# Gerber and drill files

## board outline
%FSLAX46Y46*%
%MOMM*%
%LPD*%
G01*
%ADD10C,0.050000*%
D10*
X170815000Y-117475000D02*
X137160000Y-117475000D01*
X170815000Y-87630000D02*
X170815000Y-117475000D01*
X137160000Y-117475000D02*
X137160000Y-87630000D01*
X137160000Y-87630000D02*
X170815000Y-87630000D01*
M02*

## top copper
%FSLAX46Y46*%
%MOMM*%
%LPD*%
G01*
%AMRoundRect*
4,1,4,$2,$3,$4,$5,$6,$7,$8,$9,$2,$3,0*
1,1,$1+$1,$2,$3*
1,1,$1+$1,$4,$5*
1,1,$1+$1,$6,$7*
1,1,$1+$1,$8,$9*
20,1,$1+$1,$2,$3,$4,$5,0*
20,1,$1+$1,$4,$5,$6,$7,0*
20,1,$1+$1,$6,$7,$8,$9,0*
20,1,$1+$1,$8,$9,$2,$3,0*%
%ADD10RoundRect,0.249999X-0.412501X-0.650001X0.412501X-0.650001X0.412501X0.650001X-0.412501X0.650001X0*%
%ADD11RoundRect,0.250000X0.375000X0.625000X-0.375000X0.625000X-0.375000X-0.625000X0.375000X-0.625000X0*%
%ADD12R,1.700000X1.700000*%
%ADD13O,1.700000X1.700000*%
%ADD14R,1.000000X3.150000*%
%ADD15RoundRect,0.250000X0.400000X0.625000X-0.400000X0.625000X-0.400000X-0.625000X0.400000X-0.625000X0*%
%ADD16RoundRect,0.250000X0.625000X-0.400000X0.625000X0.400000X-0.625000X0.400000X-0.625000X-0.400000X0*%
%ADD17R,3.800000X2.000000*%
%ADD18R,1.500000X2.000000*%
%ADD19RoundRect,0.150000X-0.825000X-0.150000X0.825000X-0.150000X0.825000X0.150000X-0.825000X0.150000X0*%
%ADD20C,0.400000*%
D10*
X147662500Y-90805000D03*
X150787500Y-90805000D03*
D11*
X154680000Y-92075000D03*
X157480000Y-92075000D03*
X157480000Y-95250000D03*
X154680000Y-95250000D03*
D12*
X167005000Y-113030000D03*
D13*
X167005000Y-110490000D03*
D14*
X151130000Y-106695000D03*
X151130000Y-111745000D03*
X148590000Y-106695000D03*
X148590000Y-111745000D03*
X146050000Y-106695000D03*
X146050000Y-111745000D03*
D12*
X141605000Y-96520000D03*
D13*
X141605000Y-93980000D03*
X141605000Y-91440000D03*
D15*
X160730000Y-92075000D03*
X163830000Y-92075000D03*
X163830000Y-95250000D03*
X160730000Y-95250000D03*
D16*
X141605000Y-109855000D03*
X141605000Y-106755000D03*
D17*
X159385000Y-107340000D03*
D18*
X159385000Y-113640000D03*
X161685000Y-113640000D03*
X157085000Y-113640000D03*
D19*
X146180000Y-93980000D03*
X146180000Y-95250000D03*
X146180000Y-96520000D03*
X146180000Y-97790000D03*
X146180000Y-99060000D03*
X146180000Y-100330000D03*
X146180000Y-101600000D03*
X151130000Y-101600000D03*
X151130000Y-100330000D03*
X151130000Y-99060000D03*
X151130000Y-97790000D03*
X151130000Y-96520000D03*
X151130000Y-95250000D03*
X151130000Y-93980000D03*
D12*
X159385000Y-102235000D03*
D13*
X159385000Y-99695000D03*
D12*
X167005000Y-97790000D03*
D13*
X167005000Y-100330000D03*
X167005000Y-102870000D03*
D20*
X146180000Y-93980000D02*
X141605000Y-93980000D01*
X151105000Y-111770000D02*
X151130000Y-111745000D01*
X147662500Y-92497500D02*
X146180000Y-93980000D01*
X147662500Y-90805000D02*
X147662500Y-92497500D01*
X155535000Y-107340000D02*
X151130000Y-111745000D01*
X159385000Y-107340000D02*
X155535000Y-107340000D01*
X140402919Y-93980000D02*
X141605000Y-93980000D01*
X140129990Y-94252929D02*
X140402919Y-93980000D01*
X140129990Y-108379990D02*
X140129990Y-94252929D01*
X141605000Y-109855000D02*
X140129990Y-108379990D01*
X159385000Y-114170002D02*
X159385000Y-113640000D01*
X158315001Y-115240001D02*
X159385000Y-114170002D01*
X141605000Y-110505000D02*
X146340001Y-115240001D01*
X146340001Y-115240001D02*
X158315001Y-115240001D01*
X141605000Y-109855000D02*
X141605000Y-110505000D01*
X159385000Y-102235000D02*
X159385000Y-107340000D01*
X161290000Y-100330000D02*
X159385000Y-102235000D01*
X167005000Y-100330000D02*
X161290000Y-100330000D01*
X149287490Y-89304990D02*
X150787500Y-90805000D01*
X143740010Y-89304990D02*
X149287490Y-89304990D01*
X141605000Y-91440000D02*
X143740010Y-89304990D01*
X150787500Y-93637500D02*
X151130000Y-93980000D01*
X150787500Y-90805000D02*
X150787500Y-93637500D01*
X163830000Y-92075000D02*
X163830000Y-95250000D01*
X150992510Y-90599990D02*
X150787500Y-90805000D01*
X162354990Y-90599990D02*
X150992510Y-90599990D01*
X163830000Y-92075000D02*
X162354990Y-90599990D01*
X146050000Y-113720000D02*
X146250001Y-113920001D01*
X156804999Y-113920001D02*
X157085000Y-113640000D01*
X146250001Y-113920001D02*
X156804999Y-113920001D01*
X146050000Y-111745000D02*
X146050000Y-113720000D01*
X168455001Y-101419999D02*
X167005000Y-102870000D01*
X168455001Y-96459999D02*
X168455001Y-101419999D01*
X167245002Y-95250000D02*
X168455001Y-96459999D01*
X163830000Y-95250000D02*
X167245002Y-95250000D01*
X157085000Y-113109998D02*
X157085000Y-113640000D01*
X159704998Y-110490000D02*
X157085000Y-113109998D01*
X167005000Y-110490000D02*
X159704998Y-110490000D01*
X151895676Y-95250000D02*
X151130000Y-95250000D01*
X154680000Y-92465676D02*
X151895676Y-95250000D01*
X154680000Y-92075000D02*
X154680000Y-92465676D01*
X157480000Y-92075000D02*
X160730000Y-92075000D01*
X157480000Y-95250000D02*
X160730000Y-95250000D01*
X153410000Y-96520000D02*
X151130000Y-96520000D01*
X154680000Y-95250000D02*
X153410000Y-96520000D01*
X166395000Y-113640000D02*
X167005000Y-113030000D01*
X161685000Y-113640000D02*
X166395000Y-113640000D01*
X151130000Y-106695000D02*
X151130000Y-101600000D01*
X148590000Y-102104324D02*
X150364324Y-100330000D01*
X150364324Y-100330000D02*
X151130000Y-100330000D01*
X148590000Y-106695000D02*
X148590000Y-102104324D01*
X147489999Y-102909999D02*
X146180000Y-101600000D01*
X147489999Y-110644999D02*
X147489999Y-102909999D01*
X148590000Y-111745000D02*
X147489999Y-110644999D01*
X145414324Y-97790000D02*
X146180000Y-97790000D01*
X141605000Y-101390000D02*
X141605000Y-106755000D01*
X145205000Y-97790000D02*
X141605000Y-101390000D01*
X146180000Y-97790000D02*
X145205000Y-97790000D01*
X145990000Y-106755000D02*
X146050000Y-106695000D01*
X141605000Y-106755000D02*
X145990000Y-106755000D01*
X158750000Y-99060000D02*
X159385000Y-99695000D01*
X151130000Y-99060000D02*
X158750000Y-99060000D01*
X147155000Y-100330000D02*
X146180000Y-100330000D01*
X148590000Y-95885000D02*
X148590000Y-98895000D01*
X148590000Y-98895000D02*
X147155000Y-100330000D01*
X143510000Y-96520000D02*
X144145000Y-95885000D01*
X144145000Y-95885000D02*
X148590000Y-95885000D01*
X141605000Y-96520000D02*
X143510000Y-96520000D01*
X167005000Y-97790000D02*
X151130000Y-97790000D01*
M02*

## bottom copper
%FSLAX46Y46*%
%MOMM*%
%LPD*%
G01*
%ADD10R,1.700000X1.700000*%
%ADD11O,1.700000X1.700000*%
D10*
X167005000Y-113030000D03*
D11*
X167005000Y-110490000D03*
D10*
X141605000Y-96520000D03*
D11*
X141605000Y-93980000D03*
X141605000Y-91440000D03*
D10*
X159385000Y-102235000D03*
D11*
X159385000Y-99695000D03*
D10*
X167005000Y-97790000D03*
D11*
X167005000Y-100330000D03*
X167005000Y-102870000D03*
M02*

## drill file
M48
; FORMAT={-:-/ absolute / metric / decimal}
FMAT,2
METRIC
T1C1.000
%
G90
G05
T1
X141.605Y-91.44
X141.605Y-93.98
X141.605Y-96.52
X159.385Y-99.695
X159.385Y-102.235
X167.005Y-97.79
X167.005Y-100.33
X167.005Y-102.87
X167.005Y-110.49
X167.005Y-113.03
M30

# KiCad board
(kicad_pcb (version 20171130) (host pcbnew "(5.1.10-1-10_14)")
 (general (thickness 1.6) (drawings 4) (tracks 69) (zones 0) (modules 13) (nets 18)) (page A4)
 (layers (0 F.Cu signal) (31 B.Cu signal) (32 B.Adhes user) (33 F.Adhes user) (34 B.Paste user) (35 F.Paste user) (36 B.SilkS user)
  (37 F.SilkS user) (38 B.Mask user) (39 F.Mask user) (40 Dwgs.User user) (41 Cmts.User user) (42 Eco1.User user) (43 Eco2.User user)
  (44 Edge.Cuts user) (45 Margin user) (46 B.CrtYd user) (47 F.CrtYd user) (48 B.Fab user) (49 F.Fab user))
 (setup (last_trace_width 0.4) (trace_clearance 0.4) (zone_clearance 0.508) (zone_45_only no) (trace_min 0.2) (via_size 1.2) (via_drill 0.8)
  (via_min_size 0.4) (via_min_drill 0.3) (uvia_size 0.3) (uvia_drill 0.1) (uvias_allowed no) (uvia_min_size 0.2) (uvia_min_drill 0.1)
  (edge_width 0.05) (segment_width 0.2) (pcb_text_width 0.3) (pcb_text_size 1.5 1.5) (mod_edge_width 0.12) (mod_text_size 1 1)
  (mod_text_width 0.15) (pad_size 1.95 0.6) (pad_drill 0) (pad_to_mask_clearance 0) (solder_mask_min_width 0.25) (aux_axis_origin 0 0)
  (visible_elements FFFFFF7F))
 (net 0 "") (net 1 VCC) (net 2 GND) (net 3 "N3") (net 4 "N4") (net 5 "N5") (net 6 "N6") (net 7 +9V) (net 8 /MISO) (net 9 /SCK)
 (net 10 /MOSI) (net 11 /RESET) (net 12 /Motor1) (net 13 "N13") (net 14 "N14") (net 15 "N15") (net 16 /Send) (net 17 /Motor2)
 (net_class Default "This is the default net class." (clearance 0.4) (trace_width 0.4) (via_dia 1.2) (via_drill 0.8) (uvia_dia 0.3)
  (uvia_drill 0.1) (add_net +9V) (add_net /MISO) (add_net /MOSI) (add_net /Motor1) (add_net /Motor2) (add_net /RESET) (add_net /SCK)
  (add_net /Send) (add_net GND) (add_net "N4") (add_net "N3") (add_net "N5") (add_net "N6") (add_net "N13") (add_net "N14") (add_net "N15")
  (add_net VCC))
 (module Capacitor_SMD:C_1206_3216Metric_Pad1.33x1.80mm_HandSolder (layer F.Cu) (at 149.225 90.805)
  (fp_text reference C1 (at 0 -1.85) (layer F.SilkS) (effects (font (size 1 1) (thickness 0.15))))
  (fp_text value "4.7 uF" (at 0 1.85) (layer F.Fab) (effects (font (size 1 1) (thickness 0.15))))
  (pad 1 smd roundrect (at -1.5625 0) (size 1.325 1.8) (layers F.Cu F.Paste F.Mask) (roundrect_rratio 0.1886784905660377) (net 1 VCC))
  (pad 2 smd roundrect (at 1.5625 0) (size 1.325 1.8) (layers F.Cu F.Paste F.Mask) (roundrect_rratio 0.1886784905660377) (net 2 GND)))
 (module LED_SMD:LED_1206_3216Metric (layer F.Cu) (at 156.08 92.075 180)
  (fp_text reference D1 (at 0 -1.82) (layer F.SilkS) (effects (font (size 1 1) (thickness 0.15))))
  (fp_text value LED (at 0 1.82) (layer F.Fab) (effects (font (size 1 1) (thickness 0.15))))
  (pad 2 smd roundrect (at 1.4 0 180) (size 1.25 1.75) (layers F.Cu F.Paste F.Mask) (roundrect_rratio 0.2) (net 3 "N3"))
  (pad 1 smd roundrect (at -1.4 0 180) (size 1.25 1.75) (layers F.Cu F.Paste F.Mask) (roundrect_rratio 0.2) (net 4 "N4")))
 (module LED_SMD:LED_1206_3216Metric (layer F.Cu) (at 156.08 95.25 180)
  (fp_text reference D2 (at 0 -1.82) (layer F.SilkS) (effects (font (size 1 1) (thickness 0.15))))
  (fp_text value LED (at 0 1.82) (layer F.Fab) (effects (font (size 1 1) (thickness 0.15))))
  (pad 1 smd roundrect (at -1.4 0 180) (size 1.25 1.75) (layers F.Cu F.Paste F.Mask) (roundrect_rratio 0.2) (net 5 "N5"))
  (pad 2 smd roundrect (at 1.4 0 180) (size 1.25 1.75) (layers F.Cu F.Paste F.Mask) (roundrect_rratio 0.2) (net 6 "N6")))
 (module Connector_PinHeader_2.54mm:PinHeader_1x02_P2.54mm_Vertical (layer F.Cu) (at 167.005 113.03 180)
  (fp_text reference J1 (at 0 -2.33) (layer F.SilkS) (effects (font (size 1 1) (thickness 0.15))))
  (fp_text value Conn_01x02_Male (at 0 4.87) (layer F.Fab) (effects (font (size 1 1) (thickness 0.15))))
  (pad 1 thru_hole rect (at 0 0 180) (size 1.7 1.7) (drill 1) (layers *.Cu *.Mask) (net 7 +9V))
  (pad 2 thru_hole oval (at 0 2.54 180) (size 1.7 1.7) (drill 1) (layers *.Cu *.Mask) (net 2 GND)))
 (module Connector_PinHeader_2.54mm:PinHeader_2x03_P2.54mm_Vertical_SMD (layer F.Cu) (at 148.59 109.22 270)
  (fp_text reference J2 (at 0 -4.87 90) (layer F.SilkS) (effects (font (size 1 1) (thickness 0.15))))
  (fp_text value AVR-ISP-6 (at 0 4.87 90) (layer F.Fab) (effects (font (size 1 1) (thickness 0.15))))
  (pad 1 smd rect (at -2.525 -2.54 270) (size 3.15 1) (layers F.Cu F.Paste F.Mask) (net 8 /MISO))
  (pad 2 smd rect (at 2.525 -2.54 270) (size 3.15 1) (layers F.Cu F.Paste F.Mask) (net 1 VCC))
  (pad 3 smd rect (at -2.525 0 270) (size 3.15 1) (layers F.Cu F.Paste F.Mask) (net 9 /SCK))
  (pad 4 smd rect (at 2.525 0 270) (size 3.15 1) (layers F.Cu F.Paste F.Mask) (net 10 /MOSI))
  (pad 5 smd rect (at -2.525 2.54 270) (size 3.15 1) (layers F.Cu F.Paste F.Mask) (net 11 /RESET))
  (pad 6 smd rect (at 2.525 2.54 270) (size 3.15 1) (layers F.Cu F.Paste F.Mask) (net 2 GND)))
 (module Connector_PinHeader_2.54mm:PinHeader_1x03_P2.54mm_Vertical (layer F.Cu) (at 141.605 96.52 180)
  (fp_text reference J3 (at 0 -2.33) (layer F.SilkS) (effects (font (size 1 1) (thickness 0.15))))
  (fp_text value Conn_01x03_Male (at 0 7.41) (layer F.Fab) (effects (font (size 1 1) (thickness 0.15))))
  (pad 1 thru_hole rect (at 0 0 180) (size 1.7 1.7) (drill 1) (layers *.Cu *.Mask) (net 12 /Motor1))
  (pad 2 thru_hole oval (at 0 2.54 180) (size 1.7 1.7) (drill 1) (layers *.Cu *.Mask) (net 1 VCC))
  (pad 3 thru_hole oval (at 0 5.08 180) (size 1.7 1.7) (drill 1) (layers *.Cu *.Mask) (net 2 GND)))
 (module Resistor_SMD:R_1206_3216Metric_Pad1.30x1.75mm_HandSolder (layer F.Cu) (at 162.28 92.075 180)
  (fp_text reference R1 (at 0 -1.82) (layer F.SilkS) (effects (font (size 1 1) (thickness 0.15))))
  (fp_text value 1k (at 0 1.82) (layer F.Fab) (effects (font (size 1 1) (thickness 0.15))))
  (pad 2 smd roundrect (at 1.55 0 180) (size 1.3 1.75) (layers F.Cu F.Paste F.Mask) (roundrect_rratio 0.1923076923076923) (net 4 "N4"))
  (pad 1 smd roundrect (at -1.55 0 180) (size 1.3 1.75) (layers F.Cu F.Paste F.Mask) (roundrect_rratio 0.1923076923076923) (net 2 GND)))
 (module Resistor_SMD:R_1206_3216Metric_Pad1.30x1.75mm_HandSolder (layer F.Cu) (at 162.28 95.25 180)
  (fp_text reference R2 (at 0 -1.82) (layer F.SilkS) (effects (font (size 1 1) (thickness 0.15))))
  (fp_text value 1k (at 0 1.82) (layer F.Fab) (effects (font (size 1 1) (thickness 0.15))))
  (pad 1 smd roundrect (at -1.55 0 180) (size 1.3 1.75) (layers F.Cu F.Paste F.Mask) (roundrect_rratio 0.1923076923076923) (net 2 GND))
  (pad 2 smd roundrect (at 1.55 0 180) (size 1.3 1.75) (layers F.Cu F.Paste F.Mask) (roundrect_rratio 0.1923076923076923) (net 5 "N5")))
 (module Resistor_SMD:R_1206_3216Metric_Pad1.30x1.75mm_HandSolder (layer F.Cu) (at 141.605 108.305 90)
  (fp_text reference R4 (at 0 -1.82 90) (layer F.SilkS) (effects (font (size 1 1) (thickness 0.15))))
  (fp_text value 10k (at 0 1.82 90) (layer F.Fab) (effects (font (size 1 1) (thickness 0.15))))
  (pad 1 smd roundrect (at -1.55 0 90) (size 1.3 1.75) (layers F.Cu F.Paste F.Mask) (roundrect_rratio 0.1923076923076923) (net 1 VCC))
  (pad 2 smd roundrect (at 1.55 0 90) (size 1.3 1.75) (layers F.Cu F.Paste F.Mask) (roundrect_rratio 0.1923076923076923) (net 11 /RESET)))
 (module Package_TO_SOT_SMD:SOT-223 (layer F.Cu) (at 159.385 110.49 90)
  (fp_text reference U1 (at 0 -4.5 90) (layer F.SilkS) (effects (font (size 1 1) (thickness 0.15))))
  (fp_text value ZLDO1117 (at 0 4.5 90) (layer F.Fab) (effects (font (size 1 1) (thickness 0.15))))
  (pad 4 smd rect (at 3.15 0 90) (size 2 3.8) (layers F.Cu F.Paste F.Mask) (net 1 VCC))
  (pad 2 smd rect (at -3.15 0 90) (size 2 1.5) (layers F.Cu F.Paste F.Mask) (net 1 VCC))
  (pad 3 smd rect (at -3.15 2.3 90) (size 2 1.5) (layers F.Cu F.Paste F.Mask) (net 7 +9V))
  (pad 1 smd rect (at -3.15 -2.3 90) (size 2 1.5) (layers F.Cu F.Paste F.Mask) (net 2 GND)))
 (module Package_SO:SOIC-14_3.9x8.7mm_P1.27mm (layer F.Cu) (at 148.655 97.79)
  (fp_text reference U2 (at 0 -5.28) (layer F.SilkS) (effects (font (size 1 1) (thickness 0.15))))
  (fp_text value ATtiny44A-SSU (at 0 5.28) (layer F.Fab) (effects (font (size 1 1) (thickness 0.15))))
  (pad 1 smd roundrect (at -2.475 -3.81) (size 1.95 0.6) (layers F.Cu F.Paste F.Mask) (roundrect_rratio 0.25) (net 1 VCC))
  (pad 2 smd roundrect (at -2.475 -2.54) (size 1.95 0.6) (layers F.Cu F.Paste F.Mask) (roundrect_rratio 0.25) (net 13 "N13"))
  (pad 3 smd roundrect (at -2.475 -1.27) (size 1.95 0.6) (layers F.Cu F.Paste F.Mask) (roundrect_rratio 0.25) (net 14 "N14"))
  (pad 4 smd roundrect (at -2.475 0) (size 1.95 0.6) (layers F.Cu F.Paste F.Mask) (roundrect_rratio 0.25) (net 11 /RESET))
  (pad 5 smd roundrect (at -2.475 1.27) (size 1.95 0.6) (layers F.Cu F.Paste F.Mask) (roundrect_rratio 0.25) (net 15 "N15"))
  (pad 6 smd roundrect (at -2.475 2.54) (size 1.95 0.6) (layers F.Cu F.Paste F.Mask) (roundrect_rratio 0.25) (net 12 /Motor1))
  (pad 7 smd roundrect (at -2.475 3.81) (size 1.95 0.6) (layers F.Cu F.Paste F.Mask) (roundrect_rratio 0.25) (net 10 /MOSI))
  (pad 8 smd roundrect (at 2.475 3.81) (size 1.95 0.6) (layers F.Cu F.Paste F.Mask) (roundrect_rratio 0.25) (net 8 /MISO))
  (pad 9 smd roundrect (at 2.475 2.54) (size 1.95 0.6) (layers F.Cu F.Paste F.Mask) (roundrect_rratio 0.25) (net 9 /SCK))
  (pad 10 smd roundrect (at 2.475 1.27) (size 1.95 0.6) (layers F.Cu F.Paste F.Mask) (roundrect_rratio 0.25) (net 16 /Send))
  (pad 11 smd roundrect (at 2.475 0) (size 1.95 0.6) (layers F.Cu F.Paste F.Mask) (roundrect_rratio 0.25) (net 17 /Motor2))
  (pad 12 smd roundrect (at 2.475 -1.27) (size 1.95 0.6) (layers F.Cu F.Paste F.Mask) (roundrect_rratio 0.25) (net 6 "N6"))
  (pad 13 smd roundrect (at 2.475 -2.54) (size 1.95 0.6) (layers F.Cu F.Paste F.Mask) (roundrect_rratio 0.25) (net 3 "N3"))
  (pad 14 smd roundrect (at 2.475 -3.81) (size 1.95 0.6) (layers F.Cu F.Paste F.Mask) (roundrect_rratio 0.25) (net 2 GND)))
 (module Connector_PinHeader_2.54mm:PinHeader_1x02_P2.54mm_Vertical (layer F.Cu) (at 159.385 102.235 180)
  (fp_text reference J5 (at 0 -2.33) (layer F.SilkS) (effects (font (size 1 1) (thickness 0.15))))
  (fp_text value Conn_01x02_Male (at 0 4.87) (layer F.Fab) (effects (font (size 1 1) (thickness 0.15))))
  (pad 1 thru_hole rect (at 0 0 180) (size 1.7 1.7) (drill 1) (layers *.Cu *.Mask) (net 1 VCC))
  (pad 2 thru_hole oval (at 0 2.54 180) (size 1.7 1.7) (drill 1) (layers *.Cu *.Mask) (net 16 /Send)))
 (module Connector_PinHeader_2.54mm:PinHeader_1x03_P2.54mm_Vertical (layer F.Cu) (at 167.005 97.79)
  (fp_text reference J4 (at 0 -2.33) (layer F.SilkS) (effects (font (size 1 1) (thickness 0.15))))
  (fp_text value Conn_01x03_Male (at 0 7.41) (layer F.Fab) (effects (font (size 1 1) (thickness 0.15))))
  (pad 1 thru_hole rect (at 0 0) (size 1.7 1.7) (drill 1) (layers *.Cu *.Mask) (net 17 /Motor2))
  (pad 2 thru_hole oval (at 0 2.54) (size 1.7 1.7) (drill 1) (layers *.Cu *.Mask) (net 1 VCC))
  (pad 3 thru_hole oval (at 0 5.08) (size 1.7 1.7) (drill 1) (layers *.Cu *.Mask) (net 2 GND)))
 (gr_line (start 170.815 117.475) (end 137.16 117.475) (layer Edge.Cuts) (width 0.05))
 (gr_line (start 170.815 87.63) (end 170.815 117.475) (layer Edge.Cuts) (width 0.05))
 (gr_line (start 137.16 117.475) (end 137.16 87.63) (layer Edge.Cuts) (width 0.05))
 (gr_line (start 137.16 87.63) (end 170.815 87.63) (layer Edge.Cuts) (width 0.05))
 (segment (start 146.18 93.98) (end 141.605 93.98) (width 0.4) (layer F.Cu) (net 1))
 (segment (start 151.105 111.77) (end 151.13 111.745) (width 0.4) (layer F.Cu) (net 1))
 (segment (start 147.6625 92.4975) (end 146.18 93.98) (width 0.4) (layer F.Cu) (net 1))
 (segment (start 147.6625 90.805) (end 147.6625 92.4975) (width 0.4) (layer F.Cu) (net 1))
 (segment (start 155.535 107.34) (end 151.13 111.745) (width 0.4) (layer F.Cu) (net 1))
 (segment (start 159.385 107.34) (end 155.535 107.34) (width 0.4) (layer F.Cu) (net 1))
 (segment (start 140.402919 93.98) (end 141.605 93.98) (width 0.4) (layer F.Cu) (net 1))
 (segment (start 140.12999 94.252929) (end 140.402919 93.98) (width 0.4) (layer F.Cu) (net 1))
 (segment (start 140.12999 108.37999) (end 140.12999 94.252929) (width 0.4) (layer F.Cu) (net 1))
 (segment (start 141.605 109.855) (end 140.12999 108.37999) (width 0.4) (layer F.Cu) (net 1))
 (segment (start 159.385 114.170002) (end 159.385 113.64) (width 0.4) (layer F.Cu) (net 1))
 (segment (start 158.315001 115.240001) (end 159.385 114.170002) (width 0.4) (layer F.Cu) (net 1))
 (segment (start 141.605 110.505) (end 146.340001 115.240001) (width 0.4) (layer F.Cu) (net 1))
 (segment (start 146.340001 115.240001) (end 158.315001 115.240001) (width 0.4) (layer F.Cu) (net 1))
 (segment (start 141.605 109.855) (end 141.605 110.505) (width 0.4) (layer F.Cu) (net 1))
 (segment (start 159.385 102.235) (end 159.385 107.34) (width 0.4) (layer F.Cu) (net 1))
 (segment (start 161.29 100.33) (end 159.385 102.235) (width 0.4) (layer F.Cu) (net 1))
 (segment (start 167.005 100.33) (end 161.29 100.33) (width 0.4) (layer F.Cu) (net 1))
 (segment (start 149.28749 89.30499) (end 150.7875 90.805) (width 0.4) (layer F.Cu) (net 2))
 (segment (start 143.74001 89.30499) (end 149.28749 89.30499) (width 0.4) (layer F.Cu) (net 2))
 (segment (start 141.605 91.44) (end 143.74001 89.30499) (width 0.4) (layer F.Cu) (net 2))
 (segment (start 150.7875 93.6375) (end 151.13 93.98) (width 0.4) (layer F.Cu) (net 2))
 (segment (start 150.7875 90.805) (end 150.7875 93.6375) (width 0.4) (layer F.Cu) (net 2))
 (segment (start 163.83 92.075) (end 163.83 95.25) (width 0.4) (layer F.Cu) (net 2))
 (segment (start 150.99251 90.59999) (end 150.7875 90.805) (width 0.4) (layer F.Cu) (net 2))
 (segment (start 162.35499 90.59999) (end 150.99251 90.59999) (width 0.4) (layer F.Cu) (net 2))
 (segment (start 163.83 92.075) (end 162.35499 90.59999) (width 0.4) (layer F.Cu) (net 2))
 (segment (start 146.05 113.72) (end 146.250001 113.920001) (width 0.4) (layer F.Cu) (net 2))
 (segment (start 156.804999 113.920001) (end 157.085 113.64) (width 0.4) (layer F.Cu) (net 2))
 (segment (start 146.250001 113.920001) (end 156.804999 113.920001) (width 0.4) (layer F.Cu) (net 2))
 (segment (start 146.05 111.745) (end 146.05 113.72) (width 0.4) (layer F.Cu) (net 2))
 (segment (start 168.455001 101.419999) (end 167.005 102.87) (width 0.4) (layer F.Cu) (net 2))
 (segment (start 168.455001 96.459999) (end 168.455001 101.419999) (width 0.4) (layer F.Cu) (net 2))
 (segment (start 167.245002 95.25) (end 168.455001 96.459999) (width 0.4) (layer F.Cu) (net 2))
 (segment (start 163.83 95.25) (end 167.245002 95.25) (width 0.4) (layer F.Cu) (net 2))
 (segment (start 157.085 113.109998) (end 157.085 113.64) (width 0.4) (layer F.Cu) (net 2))
 (segment (start 159.704998 110.49) (end 157.085 113.109998) (width 0.4) (layer F.Cu) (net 2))
 (segment (start 167.005 110.49) (end 159.704998 110.49) (width 0.4) (layer F.Cu) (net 2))
 (segment (start 151.895676 95.25) (end 151.13 95.25) (width 0.4) (layer F.Cu) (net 3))
 (segment (start 154.68 92.465676) (end 151.895676 95.25) (width 0.4) (layer F.Cu) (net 3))
 (segment (start 154.68 92.075) (end 154.68 92.465676) (width 0.4) (layer F.Cu) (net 3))
 (segment (start 157.48 92.075) (end 160.73 92.075) (width 0.4) (layer F.Cu) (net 4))
 (segment (start 157.48 95.25) (end 160.73 95.25) (width 0.4) (layer F.Cu) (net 5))
 (segment (start 153.41 96.52) (end 151.13 96.52) (width 0.4) (layer F.Cu) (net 6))
 (segment (start 154.68 95.25) (end 153.41 96.52) (width 0.4) (layer F.Cu) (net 6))
 (segment (start 166.395 113.64) (end 167.005 113.03) (width 0.4) (layer F.Cu) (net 7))
 (segment (start 161.685 113.64) (end 166.395 113.64) (width 0.4) (layer F.Cu) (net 7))
 (segment (start 151.13 106.695) (end 151.13 101.6) (width 0.4) (layer F.Cu) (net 8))
 (segment (start 148.59 102.104324) (end 150.364324 100.33) (width 0.4) (layer F.Cu) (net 9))
 (segment (start 150.364324 100.33) (end 151.13 100.33) (width 0.4) (layer F.Cu) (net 9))
 (segment (start 148.59 106.695) (end 148.59 102.104324) (width 0.4) (layer F.Cu) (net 9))
 (segment (start 147.489999 102.909999) (end 146.18 101.6) (width 0.4) (layer F.Cu) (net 10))
 (segment (start 147.489999 110.644999) (end 147.489999 102.909999) (width 0.4) (layer F.Cu) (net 10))
 (segment (start 148.59 111.745) (end 147.489999 110.644999) (width 0.4) (layer F.Cu) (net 10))
 (segment (start 145.414324 97.79) (end 146.18 97.79) (width 0.4) (layer F.Cu) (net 11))
 (segment (start 141.605 101.39) (end 141.605 106.755) (width 0.4) (layer F.Cu) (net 11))
 (segment (start 145.205 97.79) (end 141.605 101.39) (width 0.4) (layer F.Cu) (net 11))
 (segment (start 146.18 97.79) (end 145.205 97.79) (width 0.4) (layer F.Cu) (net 11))
 (segment (start 145.99 106.755) (end 146.05 106.695) (width 0.4) (layer F.Cu) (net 11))
 (segment (start 141.605 106.755) (end 145.99 106.755) (width 0.4) (layer F.Cu) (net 11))
 (segment (start 158.75 99.06) (end 159.385 99.695) (width 0.4) (layer F.Cu) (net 16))
 (segment (start 151.13 99.06) (end 158.75 99.06) (width 0.4) (layer F.Cu) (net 16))
 (segment (start 147.155 100.33) (end 146.18 100.33) (width 0.4) (layer F.Cu) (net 12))
 (segment (start 148.59 95.885) (end 148.59 98.895) (width 0.4) (layer F.Cu) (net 12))
 (segment (start 148.59 98.895) (end 147.155 100.33) (width 0.4) (layer F.Cu) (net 12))
 (segment (start 143.51 96.52) (end 144.145 95.885) (width 0.4) (layer F.Cu) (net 12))
 (segment (start 144.145 95.885) (end 148.59 95.885) (width 0.4) (layer F.Cu) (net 12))
 (segment (start 141.605 96.52) (end 143.51 96.52) (width 0.4) (layer F.Cu) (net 12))
 (segment (start 167.005 97.79) (end 151.13 97.79) (width 0.4) (layer F.Cu) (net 17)))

